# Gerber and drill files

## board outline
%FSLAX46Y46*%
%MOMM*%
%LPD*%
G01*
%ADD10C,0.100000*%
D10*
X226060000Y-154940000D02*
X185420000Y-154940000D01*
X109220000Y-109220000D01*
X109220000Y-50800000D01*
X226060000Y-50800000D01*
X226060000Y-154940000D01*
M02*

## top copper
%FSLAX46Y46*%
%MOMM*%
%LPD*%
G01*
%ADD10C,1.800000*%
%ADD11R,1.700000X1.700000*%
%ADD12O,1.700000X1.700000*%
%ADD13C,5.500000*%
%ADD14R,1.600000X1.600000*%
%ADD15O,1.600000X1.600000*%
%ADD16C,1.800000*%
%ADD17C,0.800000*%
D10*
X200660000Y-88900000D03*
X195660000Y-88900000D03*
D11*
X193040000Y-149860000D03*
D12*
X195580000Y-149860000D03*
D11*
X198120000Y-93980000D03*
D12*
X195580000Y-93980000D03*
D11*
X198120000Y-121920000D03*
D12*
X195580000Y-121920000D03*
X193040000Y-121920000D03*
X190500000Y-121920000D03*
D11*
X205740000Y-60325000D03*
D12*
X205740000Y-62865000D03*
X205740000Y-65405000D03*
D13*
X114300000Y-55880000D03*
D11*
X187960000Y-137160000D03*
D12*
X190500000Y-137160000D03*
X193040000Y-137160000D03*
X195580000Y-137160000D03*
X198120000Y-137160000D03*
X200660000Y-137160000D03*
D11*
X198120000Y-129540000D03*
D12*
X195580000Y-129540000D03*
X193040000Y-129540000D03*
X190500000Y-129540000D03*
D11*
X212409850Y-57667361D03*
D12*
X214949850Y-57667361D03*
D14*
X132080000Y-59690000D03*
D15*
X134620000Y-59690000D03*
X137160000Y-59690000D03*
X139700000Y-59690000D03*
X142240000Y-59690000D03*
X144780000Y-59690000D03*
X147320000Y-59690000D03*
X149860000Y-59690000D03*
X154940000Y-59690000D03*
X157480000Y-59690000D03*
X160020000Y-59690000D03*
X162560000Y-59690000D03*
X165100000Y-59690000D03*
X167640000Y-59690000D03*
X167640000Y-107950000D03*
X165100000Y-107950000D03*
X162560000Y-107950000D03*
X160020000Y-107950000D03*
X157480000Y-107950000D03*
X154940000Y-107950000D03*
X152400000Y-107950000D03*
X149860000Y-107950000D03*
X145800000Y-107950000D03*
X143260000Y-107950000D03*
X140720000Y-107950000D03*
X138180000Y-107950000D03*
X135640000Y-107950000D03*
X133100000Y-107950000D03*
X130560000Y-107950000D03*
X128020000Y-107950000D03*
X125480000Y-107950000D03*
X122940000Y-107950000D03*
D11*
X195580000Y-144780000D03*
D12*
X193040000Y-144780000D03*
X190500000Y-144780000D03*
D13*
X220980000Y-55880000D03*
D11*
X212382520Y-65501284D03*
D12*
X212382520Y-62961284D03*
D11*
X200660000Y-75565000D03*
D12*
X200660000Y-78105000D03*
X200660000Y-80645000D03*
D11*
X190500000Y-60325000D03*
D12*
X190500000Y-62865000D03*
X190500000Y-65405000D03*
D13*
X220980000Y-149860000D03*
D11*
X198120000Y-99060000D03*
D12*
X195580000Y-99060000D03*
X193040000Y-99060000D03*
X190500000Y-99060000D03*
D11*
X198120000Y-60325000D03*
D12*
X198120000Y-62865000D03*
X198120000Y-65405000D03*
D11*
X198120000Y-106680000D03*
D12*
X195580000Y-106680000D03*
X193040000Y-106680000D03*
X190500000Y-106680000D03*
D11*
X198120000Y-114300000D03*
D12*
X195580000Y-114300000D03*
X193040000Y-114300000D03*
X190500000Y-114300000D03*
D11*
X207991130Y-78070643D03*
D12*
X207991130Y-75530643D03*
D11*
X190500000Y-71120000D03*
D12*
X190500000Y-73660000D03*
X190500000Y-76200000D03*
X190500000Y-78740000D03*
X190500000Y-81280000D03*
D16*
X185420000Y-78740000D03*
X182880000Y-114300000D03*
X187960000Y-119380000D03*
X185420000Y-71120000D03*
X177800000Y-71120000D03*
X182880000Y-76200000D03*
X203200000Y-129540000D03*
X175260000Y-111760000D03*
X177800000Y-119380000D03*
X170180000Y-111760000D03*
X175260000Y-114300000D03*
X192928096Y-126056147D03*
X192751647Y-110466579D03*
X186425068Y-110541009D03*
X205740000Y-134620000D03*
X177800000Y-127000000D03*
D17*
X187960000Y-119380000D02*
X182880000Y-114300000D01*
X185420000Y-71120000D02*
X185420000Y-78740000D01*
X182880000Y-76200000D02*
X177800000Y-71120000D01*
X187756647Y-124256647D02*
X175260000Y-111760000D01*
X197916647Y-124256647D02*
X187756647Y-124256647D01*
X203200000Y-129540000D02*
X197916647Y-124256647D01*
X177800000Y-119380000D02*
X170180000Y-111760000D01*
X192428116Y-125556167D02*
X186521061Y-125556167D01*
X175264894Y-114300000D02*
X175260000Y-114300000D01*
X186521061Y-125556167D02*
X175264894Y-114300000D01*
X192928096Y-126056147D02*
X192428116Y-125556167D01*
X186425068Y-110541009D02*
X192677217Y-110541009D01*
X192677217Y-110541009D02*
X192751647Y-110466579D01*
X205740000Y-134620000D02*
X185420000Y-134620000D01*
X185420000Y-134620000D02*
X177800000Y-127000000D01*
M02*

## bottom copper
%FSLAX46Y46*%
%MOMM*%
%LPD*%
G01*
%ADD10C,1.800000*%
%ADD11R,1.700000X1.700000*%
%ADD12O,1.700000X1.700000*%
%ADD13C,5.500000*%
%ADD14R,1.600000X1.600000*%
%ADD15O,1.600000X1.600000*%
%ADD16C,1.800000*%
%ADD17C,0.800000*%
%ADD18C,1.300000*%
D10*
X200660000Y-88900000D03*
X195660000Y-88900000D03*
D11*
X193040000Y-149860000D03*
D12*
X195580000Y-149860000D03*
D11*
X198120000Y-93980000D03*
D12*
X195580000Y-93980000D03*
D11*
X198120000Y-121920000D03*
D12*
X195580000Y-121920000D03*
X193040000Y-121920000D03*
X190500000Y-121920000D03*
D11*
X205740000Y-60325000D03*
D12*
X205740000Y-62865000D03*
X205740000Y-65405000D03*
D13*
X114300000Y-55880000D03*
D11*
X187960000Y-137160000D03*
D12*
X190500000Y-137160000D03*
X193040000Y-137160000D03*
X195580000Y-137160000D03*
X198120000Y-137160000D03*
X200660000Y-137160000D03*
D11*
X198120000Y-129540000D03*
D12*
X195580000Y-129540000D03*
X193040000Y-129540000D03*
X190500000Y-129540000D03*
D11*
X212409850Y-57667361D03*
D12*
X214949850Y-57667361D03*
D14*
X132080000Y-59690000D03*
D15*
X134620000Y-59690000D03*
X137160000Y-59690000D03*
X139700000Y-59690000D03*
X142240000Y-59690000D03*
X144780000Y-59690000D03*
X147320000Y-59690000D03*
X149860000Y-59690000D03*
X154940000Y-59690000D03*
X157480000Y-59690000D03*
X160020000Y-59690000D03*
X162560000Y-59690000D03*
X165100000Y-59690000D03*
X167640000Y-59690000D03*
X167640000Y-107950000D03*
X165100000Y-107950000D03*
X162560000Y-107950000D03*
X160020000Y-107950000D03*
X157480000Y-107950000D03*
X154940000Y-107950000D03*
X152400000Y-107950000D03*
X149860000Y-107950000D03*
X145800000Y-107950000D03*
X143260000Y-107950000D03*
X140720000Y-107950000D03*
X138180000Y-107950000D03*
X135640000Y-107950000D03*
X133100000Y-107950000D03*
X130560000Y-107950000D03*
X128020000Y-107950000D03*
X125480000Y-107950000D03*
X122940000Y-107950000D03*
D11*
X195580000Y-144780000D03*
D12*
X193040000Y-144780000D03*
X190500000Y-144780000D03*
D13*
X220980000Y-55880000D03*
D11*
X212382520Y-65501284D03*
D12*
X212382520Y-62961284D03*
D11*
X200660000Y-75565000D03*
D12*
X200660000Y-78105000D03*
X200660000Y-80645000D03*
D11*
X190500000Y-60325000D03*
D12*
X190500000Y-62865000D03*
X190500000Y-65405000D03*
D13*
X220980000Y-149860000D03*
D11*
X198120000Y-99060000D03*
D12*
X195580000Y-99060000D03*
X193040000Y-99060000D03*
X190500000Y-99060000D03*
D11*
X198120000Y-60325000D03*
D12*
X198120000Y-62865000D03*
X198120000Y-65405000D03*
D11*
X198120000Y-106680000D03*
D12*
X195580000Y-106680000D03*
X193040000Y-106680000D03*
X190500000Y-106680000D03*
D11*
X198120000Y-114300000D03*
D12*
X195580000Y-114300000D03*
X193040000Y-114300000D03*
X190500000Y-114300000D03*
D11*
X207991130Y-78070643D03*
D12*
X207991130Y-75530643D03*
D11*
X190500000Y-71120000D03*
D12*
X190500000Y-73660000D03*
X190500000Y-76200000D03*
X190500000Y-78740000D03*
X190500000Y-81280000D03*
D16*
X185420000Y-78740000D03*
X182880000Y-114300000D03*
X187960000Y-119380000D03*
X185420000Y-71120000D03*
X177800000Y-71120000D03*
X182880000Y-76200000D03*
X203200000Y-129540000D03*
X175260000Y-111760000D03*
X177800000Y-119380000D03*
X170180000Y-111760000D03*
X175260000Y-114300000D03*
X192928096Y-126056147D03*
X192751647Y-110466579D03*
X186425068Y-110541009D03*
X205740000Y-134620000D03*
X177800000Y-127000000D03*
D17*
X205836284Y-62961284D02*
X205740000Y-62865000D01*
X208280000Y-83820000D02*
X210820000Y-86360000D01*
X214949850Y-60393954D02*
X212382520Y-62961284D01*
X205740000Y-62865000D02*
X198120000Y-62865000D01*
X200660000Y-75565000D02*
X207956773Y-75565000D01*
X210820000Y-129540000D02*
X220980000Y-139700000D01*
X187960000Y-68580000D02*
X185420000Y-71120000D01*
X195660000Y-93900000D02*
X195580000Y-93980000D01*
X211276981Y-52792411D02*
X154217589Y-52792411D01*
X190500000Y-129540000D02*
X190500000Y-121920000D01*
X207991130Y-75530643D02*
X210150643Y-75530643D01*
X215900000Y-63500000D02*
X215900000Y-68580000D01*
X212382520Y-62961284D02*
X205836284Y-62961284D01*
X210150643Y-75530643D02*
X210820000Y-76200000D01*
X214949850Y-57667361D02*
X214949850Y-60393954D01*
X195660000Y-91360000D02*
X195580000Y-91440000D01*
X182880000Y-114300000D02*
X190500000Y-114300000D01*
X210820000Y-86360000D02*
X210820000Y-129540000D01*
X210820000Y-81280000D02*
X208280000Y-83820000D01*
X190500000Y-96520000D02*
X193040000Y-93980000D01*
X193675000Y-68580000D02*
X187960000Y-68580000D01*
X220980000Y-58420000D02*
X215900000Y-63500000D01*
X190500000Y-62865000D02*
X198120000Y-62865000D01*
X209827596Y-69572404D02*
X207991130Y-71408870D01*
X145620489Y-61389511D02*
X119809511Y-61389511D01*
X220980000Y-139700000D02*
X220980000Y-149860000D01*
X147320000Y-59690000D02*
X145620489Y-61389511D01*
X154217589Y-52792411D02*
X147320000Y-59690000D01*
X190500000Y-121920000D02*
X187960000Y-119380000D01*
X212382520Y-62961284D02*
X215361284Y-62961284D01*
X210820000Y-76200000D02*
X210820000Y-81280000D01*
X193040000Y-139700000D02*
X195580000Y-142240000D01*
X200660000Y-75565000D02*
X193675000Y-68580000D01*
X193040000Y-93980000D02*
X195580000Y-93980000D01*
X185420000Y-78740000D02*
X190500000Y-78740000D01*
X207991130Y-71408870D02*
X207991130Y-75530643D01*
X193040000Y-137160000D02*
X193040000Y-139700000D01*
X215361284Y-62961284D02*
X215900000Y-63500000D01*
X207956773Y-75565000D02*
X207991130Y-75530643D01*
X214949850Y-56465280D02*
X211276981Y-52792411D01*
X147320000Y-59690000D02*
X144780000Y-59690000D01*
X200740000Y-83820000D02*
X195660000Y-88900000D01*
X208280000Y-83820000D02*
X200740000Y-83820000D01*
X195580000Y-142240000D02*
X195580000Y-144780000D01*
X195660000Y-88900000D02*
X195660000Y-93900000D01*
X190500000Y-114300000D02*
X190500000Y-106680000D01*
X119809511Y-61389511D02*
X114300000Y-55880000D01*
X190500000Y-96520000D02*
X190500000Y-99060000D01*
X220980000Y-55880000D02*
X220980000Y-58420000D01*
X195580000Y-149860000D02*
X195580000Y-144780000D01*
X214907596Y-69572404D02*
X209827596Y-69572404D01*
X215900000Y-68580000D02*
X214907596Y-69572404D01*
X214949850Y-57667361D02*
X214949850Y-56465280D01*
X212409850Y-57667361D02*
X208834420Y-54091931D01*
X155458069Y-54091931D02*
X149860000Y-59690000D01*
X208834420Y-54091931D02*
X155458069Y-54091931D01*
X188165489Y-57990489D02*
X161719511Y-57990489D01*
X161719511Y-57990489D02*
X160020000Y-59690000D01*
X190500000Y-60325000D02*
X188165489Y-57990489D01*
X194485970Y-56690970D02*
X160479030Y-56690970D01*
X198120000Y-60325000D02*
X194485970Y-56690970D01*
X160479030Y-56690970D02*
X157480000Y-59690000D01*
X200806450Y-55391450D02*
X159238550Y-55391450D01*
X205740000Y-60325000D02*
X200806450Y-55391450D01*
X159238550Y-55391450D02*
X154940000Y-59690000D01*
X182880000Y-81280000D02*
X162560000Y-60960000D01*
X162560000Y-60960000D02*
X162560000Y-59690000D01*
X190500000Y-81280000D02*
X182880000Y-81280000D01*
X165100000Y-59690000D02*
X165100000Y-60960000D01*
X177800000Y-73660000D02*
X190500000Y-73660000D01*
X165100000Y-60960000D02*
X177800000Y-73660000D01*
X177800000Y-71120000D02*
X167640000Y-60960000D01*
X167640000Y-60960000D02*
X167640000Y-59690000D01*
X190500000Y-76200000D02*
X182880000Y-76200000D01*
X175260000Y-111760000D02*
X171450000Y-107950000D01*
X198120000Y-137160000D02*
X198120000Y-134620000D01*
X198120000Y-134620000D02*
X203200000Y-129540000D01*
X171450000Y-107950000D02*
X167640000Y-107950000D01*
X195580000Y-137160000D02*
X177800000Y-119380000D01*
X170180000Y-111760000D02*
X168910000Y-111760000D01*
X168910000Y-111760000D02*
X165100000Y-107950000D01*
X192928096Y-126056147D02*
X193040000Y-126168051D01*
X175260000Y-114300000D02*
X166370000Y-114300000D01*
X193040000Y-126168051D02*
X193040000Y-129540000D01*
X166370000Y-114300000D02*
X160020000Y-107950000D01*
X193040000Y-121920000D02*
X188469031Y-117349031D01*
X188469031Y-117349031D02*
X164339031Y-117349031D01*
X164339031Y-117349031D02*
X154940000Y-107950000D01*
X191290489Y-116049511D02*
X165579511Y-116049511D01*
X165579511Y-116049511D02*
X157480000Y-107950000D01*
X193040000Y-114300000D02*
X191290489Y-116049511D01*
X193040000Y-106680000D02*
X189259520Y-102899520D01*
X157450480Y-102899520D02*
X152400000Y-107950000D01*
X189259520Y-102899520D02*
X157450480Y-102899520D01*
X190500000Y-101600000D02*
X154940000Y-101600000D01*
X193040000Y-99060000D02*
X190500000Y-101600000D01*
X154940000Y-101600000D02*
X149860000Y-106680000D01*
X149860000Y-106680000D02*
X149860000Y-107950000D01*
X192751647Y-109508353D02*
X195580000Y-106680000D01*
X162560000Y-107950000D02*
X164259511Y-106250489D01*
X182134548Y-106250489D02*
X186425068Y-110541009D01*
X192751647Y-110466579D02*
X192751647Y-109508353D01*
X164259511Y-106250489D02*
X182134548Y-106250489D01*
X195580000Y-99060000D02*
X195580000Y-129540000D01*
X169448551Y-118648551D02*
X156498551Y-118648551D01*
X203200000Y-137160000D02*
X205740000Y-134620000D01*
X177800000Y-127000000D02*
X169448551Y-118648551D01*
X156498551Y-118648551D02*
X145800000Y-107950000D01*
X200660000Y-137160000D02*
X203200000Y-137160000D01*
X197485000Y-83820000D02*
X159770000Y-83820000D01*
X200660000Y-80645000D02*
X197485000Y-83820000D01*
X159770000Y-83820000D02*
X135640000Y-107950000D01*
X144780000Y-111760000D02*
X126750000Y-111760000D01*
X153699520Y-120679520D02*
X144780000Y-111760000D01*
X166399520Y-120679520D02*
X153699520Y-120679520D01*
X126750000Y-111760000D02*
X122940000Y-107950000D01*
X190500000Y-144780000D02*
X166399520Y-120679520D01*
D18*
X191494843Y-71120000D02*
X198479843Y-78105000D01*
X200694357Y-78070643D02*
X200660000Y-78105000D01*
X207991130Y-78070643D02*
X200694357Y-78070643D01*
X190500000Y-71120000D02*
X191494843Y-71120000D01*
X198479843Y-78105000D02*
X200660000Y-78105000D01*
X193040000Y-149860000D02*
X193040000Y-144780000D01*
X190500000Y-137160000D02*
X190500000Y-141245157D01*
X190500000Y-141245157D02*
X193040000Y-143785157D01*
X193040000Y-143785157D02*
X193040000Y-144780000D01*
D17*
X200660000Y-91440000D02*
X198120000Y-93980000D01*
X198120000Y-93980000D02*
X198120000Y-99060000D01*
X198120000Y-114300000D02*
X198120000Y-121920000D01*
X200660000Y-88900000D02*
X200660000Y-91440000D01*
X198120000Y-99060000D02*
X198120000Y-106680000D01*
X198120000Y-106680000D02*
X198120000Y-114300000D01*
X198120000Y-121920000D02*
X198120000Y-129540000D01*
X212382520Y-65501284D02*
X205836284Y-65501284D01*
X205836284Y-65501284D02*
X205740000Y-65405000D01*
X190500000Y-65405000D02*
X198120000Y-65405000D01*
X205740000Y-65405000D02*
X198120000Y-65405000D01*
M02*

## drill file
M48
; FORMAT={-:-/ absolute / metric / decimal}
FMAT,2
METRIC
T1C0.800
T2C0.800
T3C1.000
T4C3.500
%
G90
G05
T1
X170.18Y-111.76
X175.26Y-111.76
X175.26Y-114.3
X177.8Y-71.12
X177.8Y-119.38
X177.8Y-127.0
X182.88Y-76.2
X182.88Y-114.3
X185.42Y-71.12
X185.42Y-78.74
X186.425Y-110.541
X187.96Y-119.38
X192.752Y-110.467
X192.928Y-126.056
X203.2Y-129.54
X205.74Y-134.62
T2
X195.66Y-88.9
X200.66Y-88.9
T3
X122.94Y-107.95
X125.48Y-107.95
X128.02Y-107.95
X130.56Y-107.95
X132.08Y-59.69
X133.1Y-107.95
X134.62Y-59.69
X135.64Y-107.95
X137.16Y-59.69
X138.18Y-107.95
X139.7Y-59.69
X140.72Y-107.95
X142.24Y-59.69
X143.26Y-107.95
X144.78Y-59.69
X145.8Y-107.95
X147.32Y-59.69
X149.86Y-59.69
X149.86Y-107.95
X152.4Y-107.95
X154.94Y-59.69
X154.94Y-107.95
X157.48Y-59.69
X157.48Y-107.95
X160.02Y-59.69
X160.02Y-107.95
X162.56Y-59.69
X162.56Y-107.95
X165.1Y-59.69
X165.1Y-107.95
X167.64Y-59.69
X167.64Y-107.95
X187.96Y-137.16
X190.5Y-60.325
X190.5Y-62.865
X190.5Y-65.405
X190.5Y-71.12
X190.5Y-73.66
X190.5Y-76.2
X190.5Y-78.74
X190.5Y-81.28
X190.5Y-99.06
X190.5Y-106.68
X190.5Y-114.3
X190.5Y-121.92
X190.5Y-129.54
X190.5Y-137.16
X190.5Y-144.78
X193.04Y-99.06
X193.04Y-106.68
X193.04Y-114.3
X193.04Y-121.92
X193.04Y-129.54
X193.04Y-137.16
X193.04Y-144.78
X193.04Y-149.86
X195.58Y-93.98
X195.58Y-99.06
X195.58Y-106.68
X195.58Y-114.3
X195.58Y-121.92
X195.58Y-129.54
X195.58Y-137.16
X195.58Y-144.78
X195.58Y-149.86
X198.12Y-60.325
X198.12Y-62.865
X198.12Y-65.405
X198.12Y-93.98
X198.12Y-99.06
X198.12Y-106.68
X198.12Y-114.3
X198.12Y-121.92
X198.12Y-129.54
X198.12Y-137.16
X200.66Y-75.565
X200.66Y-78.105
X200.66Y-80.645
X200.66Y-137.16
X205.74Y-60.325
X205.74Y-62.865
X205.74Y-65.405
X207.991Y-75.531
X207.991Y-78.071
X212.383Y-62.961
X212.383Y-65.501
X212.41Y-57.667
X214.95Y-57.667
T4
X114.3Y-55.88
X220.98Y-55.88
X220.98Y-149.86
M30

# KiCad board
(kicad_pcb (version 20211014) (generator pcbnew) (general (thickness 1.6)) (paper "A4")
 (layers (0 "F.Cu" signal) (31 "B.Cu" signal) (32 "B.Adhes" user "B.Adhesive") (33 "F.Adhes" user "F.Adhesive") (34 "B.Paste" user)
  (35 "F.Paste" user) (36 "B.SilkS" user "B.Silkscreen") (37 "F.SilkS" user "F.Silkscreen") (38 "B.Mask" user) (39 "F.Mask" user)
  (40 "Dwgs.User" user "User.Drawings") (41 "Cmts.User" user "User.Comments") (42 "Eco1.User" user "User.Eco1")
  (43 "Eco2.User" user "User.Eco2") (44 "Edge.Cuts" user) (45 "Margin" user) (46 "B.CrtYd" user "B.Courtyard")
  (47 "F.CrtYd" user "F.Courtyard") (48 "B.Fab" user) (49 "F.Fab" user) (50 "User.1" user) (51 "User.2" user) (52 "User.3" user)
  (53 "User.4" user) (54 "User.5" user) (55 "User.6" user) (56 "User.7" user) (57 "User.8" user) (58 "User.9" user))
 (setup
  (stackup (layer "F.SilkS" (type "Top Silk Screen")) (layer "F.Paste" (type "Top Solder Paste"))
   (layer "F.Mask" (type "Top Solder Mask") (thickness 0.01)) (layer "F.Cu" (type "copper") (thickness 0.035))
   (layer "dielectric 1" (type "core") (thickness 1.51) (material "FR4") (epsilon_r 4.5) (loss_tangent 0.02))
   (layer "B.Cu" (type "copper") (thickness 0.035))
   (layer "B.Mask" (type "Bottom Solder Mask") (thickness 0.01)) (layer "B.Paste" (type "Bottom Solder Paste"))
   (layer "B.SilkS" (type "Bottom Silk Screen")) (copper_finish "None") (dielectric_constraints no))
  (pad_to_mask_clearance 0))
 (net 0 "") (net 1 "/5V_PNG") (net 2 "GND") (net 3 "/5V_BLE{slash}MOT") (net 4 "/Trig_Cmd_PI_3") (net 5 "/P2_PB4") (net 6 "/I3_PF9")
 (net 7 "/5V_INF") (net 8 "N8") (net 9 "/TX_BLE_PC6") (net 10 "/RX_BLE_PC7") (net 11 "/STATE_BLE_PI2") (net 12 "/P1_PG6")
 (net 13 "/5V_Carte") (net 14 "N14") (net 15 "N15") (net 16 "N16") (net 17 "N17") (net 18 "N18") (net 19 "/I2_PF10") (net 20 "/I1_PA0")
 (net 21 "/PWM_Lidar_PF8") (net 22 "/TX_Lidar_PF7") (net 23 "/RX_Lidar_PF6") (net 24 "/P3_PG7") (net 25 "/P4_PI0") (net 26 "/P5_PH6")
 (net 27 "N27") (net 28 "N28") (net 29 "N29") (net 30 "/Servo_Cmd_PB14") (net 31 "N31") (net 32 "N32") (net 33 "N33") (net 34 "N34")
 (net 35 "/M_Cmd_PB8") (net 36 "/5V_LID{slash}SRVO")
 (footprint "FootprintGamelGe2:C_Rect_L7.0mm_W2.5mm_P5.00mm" (layer "F.Cu") (at 200.66 88.9 180)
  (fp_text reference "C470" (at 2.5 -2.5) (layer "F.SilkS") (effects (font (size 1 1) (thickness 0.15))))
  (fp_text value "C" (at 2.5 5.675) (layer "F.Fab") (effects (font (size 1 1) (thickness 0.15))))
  (pad "1" thru_hole circle locked (at 0 0 180) (size 1.8 1.8) (drill 0.8) (layers *.Cu *.Mask) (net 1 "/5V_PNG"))
  (pad "2" thru_hole circle locked (at 5 0 180) (size 1.8 1.8) (drill 0.8) (layers *.Cu *.Mask) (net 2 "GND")))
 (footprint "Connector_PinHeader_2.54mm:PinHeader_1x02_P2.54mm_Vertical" (layer "F.Cu") (at 193.04 149.86 90)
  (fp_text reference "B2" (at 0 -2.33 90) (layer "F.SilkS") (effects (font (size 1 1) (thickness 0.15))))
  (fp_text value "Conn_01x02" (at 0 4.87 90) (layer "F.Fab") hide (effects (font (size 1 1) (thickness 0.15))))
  (pad "1" thru_hole rect (at 0 0 90) (size 1.7 1.7) (drill 1) (layers *.Cu *.Mask) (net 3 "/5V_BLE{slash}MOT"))
  (pad "2" thru_hole oval (at 0 2.54 90) (size 1.7 1.7) (drill 1) (layers *.Cu *.Mask) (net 2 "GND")))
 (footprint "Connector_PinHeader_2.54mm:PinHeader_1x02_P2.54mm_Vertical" (layer "F.Cu") (at 198.12 93.98 -90)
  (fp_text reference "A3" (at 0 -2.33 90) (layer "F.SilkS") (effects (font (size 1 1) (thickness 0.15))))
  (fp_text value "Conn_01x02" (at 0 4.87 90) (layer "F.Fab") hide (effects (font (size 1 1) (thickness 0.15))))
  (pad "1" thru_hole rect (at 0 0 270) (size 1.7 1.7) (drill 1) (layers *.Cu *.Mask) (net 1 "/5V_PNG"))
  (pad "2" thru_hole oval (at 0 2.54 270) (size 1.7 1.7) (drill 1) (layers *.Cu *.Mask) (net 2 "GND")))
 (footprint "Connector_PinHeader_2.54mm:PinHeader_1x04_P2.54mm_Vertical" (layer "F.Cu") (at 198.12 121.92 -90)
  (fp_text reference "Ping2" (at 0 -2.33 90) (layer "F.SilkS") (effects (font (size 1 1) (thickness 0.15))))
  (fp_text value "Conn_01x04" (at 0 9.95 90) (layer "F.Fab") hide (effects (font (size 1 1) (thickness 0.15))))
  (pad "1" thru_hole rect (at 0 0 270) (size 1.7 1.7) (drill 1) (layers *.Cu *.Mask) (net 1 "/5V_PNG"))
  (pad "2" thru_hole oval (at 0 2.54 270) (size 1.7 1.7) (drill 1) (layers *.Cu *.Mask) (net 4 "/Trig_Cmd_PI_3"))
  (pad "3" thru_hole oval (at 0 5.08 270) (size 1.7 1.7) (drill 1) (layers *.Cu *.Mask) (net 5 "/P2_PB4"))
  (pad "4" thru_hole oval (at 0 7.62 270) (size 1.7 1.7) (drill 1) (layers *.Cu *.Mask) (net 2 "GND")))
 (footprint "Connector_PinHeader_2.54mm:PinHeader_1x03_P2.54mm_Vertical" (layer "F.Cu") (at 205.74 60.325)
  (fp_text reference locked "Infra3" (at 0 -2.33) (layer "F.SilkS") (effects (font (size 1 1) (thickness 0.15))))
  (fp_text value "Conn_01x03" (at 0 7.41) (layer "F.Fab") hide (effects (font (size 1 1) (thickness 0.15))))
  (pad "1" thru_hole rect (at 0 0) (size 1.7 1.7) (drill 1) (layers *.Cu *.Mask) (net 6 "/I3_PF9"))
  (pad "2" thru_hole oval (at 0 2.54) (size 1.7 1.7) (drill 1) (layers *.Cu *.Mask) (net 2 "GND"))
  (pad "3" thru_hole oval (at 0 5.08) (size 1.7 1.7) (drill 1) (layers *.Cu *.Mask) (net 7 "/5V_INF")))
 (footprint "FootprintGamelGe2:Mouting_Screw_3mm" (layer "F.Cu") (at 114.3 55.88)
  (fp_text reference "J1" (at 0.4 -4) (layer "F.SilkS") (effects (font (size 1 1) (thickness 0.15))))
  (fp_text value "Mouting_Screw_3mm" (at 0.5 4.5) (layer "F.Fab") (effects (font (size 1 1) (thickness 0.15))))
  (pad "1" thru_hole circle locked (at 0 0) (size 5.5 5.5) (drill 3.5) (layers *.Cu *.Mask) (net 2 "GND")))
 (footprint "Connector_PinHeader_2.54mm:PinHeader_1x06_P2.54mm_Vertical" (layer "F.Cu") (at 187.96 137.16 90)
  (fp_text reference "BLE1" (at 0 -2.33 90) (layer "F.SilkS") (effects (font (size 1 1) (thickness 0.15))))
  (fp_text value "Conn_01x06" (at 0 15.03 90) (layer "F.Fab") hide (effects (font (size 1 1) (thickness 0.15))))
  (pad "1" thru_hole rect (at 0 0 90) (size 1.7 1.7) (drill 1) (layers *.Cu *.Mask) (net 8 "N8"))
  (pad "2" thru_hole oval (at 0 2.54 90) (size 1.7 1.7) (drill 1) (layers *.Cu *.Mask) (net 3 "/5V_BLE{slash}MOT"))
  (pad "3" thru_hole oval (at 0 5.08 90) (size 1.7 1.7) (drill 1) (layers *.Cu *.Mask) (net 2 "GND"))
  (pad "4" thru_hole oval (at 0 7.62 90) (size 1.7 1.7) (drill 1) (layers *.Cu *.Mask) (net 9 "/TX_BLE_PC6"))
  (pad "5" thru_hole oval (at 0 10.16 90) (size 1.7 1.7) (drill 1) (layers *.Cu *.Mask) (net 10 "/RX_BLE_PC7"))
  (pad "6" thru_hole oval (at 0 12.7 90) (size 1.7 1.7) (drill 1) (layers *.Cu *.Mask) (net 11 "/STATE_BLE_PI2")))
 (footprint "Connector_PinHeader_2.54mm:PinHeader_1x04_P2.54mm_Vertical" (layer "F.Cu") (at 198.12 129.54 -90)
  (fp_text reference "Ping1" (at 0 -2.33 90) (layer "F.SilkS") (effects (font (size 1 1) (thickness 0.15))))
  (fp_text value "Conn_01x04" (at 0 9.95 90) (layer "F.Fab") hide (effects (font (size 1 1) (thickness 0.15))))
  (pad "1" thru_hole rect (at 0 0 270) (size 1.7 1.7) (drill 1) (layers *.Cu *.Mask) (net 1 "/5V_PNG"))
  (pad "2" thru_hole oval (at 0 2.54 270) (size 1.7 1.7) (drill 1) (layers *.Cu *.Mask) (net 4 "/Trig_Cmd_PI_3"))
  (pad "3" thru_hole oval (at 0 5.08 270) (size 1.7 1.7) (drill 1) (layers *.Cu *.Mask) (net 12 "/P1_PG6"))
  (pad "4" thru_hole oval (at 0 7.62 270) (size 1.7 1.7) (drill 1) (layers *.Cu *.Mask) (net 2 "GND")))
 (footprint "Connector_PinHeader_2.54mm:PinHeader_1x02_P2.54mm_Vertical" (layer "F.Cu") (at 212.40985 57.667361 90)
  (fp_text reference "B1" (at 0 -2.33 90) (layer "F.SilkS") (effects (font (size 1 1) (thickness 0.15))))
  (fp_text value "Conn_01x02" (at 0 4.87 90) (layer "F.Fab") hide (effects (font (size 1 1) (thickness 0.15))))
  (pad "1" thru_hole rect (at 0 0 90) (size 1.7 1.7) (drill 1) (layers *.Cu *.Mask) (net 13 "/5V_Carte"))
  (pad "2" thru_hole oval (at 0 2.54 90) (size 1.7 1.7) (drill 1) (layers *.Cu *.Mask) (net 2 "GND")))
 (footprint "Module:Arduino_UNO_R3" (layer "F.Cu") (at 132.08 59.69)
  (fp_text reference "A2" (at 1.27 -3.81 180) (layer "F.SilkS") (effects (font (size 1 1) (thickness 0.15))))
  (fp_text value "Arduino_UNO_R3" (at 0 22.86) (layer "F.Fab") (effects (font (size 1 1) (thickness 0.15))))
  (pad "1" thru_hole rect (at 0 0 90) (size 1.6 1.6) (drill 1) (layers *.Cu *.Mask) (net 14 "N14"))
  (pad "2" thru_hole oval (at 2.54 0 90) (size 1.6 1.6) (drill 1) (layers *.Cu *.Mask) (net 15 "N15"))
  (pad "3" thru_hole oval (at 5.08 0 90) (size 1.6 1.6) (drill 1) (layers *.Cu *.Mask) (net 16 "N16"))
  (pad "4" thru_hole oval (at 7.62 0 90) (size 1.6 1.6) (drill 1) (layers *.Cu *.Mask) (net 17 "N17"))
  (pad "5" thru_hole oval (at 10.16 0 90) (size 1.6 1.6) (drill 1) (layers *.Cu *.Mask) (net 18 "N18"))
  (pad "6" thru_hole oval (at 12.7 0 90) (size 1.6 1.6) (drill 1) (layers *.Cu *.Mask) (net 2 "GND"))
  (pad "7" thru_hole oval (at 15.24 0 90) (size 1.6 1.6) (drill 1) (layers *.Cu *.Mask) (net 2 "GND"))
  (pad "8" thru_hole oval (at 17.78 0 90) (size 1.6 1.6) (drill 1) (layers *.Cu *.Mask) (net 13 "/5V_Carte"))
  (pad "9" thru_hole oval (at 22.86 0 90) (size 1.6 1.6) (drill 1) (layers *.Cu *.Mask) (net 6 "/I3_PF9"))
  (pad "10" thru_hole oval (at 25.4 0 90) (size 1.6 1.6) (drill 1) (layers *.Cu *.Mask) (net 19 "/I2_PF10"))
  (pad "11" thru_hole oval (at 27.94 0 90) (size 1.6 1.6) (drill 1) (layers *.Cu *.Mask) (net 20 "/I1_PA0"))
  (pad "12" thru_hole oval (at 30.48 0 90) (size 1.6 1.6) (drill 1) (layers *.Cu *.Mask) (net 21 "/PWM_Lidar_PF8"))
  (pad "13" thru_hole oval (at 33.02 0 90) (size 1.6 1.6) (drill 1) (layers *.Cu *.Mask) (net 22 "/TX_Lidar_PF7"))
  (pad "14" thru_hole oval (at 35.56 0 90) (size 1.6 1.6) (drill 1) (layers *.Cu *.Mask) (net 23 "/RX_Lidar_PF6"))
  (pad "15" thru_hole oval (at 35.56 48.26 90) (size 1.6 1.6) (drill 1) (layers *.Cu *.Mask) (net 10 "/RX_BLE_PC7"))
  (pad "16" thru_hole oval (at 33.02 48.26 90) (size 1.6 1.6) (drill 1) (layers *.Cu *.Mask) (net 9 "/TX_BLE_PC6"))
  (pad "17" thru_hole oval (at 30.48 48.26 90) (size 1.6 1.6) (drill 1) (layers *.Cu *.Mask) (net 4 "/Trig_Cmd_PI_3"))
  (pad "18" thru_hole oval (at 27.94 48.26 90) (size 1.6 1.6) (drill 1) (layers *.Cu *.Mask) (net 12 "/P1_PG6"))
  (pad "19" thru_hole oval (at 25.4 48.26 90) (size 1.6 1.6) (drill 1) (layers *.Cu *.Mask) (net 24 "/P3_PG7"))
  (pad "20" thru_hole oval (at 22.86 48.26 90) (size 1.6 1.6) (drill 1) (layers *.Cu *.Mask) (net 5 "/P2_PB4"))
  (pad "21" thru_hole oval (at 20.32 48.26 90) (size 1.6 1.6) (drill 1) (layers *.Cu *.Mask) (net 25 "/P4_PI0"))
  (pad "22" thru_hole oval (at 17.78 48.26 90) (size 1.6 1.6) (drill 1) (layers *.Cu *.Mask) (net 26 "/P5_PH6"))
  (pad "23" thru_hole oval (at 13.72 48.26 90) (size 1.6 1.6) (drill 1) (layers *.Cu *.Mask) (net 11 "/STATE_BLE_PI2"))
  (pad "24" thru_hole oval (at 11.18 48.26 90) (size 1.6 1.6) (drill 1) (layers *.Cu *.Mask) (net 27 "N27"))
  (pad "25" thru_hole oval (at 8.64 48.26 90) (size 1.6 1.6) (drill 1) (layers *.Cu *.Mask) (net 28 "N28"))
  (pad "26" thru_hole oval (at 6.1 48.26 90) (size 1.6 1.6) (drill 1) (layers *.Cu *.Mask) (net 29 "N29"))
  (pad "27" thru_hole oval (at 3.56 48.26 90) (size 1.6 1.6) (drill 1) (layers *.Cu *.Mask) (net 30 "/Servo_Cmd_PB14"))
  (pad "28" thru_hole oval (at 1.02 48.26 90) (size 1.6 1.6) (drill 1) (layers *.Cu *.Mask) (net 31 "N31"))
  (pad "29" thru_hole oval (at -1.52 48.26 90) (size 1.6 1.6) (drill 1) (layers *.Cu *.Mask) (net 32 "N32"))
  (pad "30" thru_hole oval (at -4.06 48.26 90) (size 1.6 1.6) (drill 1) (layers *.Cu *.Mask) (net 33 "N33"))
  (pad "31" thru_hole oval (at -6.6 48.26 90) (size 1.6 1.6) (drill 1) (layers *.Cu *.Mask) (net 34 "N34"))
  (pad "32" thru_hole oval (at -9.14 48.26 90) (size 1.6 1.6) (drill 1) (layers *.Cu *.Mask) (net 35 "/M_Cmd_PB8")))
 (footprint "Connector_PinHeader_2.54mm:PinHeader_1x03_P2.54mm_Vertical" (layer "F.Cu") (at 195.58 144.78 -90)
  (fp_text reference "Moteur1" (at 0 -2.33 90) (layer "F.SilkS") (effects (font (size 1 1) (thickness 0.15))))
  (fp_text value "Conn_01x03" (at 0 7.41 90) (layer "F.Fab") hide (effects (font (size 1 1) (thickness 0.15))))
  (pad "1" thru_hole rect (at 0 0 270) (size 1.7 1.7) (drill 1) (layers *.Cu *.Mask) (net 2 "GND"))
  (pad "2" thru_hole oval (at 0 2.54 270) (size 1.7 1.7) (drill 1) (layers *.Cu *.Mask) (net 3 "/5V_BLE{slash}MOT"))
  (pad "3" thru_hole oval (at 0 5.08 270) (size 1.7 1.7) (drill 1) (layers *.Cu *.Mask) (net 35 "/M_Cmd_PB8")))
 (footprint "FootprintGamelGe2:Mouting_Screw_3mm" (layer "F.Cu") (at 220.98 55.88)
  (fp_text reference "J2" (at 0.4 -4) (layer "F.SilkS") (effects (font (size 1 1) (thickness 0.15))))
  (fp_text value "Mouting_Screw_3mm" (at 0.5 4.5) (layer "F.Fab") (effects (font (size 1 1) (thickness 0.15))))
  (pad "1" thru_hole circle locked (at 0 0) (size 5.5 5.5) (drill 3.5) (layers *.Cu *.Mask) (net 2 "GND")))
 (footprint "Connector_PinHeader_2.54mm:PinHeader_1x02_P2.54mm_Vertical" (layer "F.Cu") (at 212.38252 65.501284 180)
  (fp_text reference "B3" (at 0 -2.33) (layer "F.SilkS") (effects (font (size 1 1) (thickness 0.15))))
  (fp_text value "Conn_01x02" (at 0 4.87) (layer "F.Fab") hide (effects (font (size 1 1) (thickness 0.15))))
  (pad "1" thru_hole rect (at 0 0 180) (size 1.7 1.7) (drill 1) (layers *.Cu *.Mask) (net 7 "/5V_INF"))
  (pad "2" thru_hole oval (at 0 2.54 180) (size 1.7 1.7) (drill 1) (layers *.Cu *.Mask) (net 2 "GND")))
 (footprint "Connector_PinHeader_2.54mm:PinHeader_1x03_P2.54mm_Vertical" (layer "F.Cu") (at 200.66 75.565)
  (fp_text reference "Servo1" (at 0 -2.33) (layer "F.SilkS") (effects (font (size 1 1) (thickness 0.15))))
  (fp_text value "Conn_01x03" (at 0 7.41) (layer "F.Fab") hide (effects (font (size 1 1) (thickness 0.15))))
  (pad "1" thru_hole rect (at 0 0) (size 1.7 1.7) (drill 1) (layers *.Cu *.Mask) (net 2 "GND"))
  (pad "2" thru_hole oval (at 0 2.54) (size 1.7 1.7) (drill 1) (layers *.Cu *.Mask) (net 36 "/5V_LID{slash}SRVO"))
  (pad "3" thru_hole oval (at 0 5.08) (size 1.7 1.7) (drill 1) (layers *.Cu *.Mask) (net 30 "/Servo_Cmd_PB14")))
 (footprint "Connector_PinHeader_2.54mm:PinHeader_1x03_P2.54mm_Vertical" (layer "F.Cu") (at 190.5 60.325)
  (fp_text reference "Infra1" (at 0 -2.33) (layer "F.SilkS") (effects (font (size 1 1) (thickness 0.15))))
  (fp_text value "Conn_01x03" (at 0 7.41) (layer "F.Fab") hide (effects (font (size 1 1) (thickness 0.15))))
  (pad "1" thru_hole rect (at 0 0) (size 1.7 1.7) (drill 1) (layers *.Cu *.Mask) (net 20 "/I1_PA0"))
  (pad "2" thru_hole oval (at 0 2.54) (size 1.7 1.7) (drill 1) (layers *.Cu *.Mask) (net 2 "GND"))
  (pad "3" thru_hole oval (at 0 5.08) (size 1.7 1.7) (drill 1) (layers *.Cu *.Mask) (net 7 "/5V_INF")))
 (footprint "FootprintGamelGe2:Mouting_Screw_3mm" (layer "F.Cu") (at 220.98 149.86)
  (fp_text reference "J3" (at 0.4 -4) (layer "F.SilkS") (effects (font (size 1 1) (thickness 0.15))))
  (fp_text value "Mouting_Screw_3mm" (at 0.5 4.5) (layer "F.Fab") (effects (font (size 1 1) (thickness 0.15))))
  (pad "1" thru_hole circle locked (at 0 0) (size 5.5 5.5) (drill 3.5) (layers *.Cu *.Mask) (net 2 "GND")))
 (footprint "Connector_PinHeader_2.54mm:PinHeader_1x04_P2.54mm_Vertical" (layer "F.Cu") (at 198.12 99.06 -90)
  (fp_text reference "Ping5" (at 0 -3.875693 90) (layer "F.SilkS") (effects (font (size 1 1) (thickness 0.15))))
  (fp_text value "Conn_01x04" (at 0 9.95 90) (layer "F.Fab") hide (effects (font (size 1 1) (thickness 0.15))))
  (pad "1" thru_hole rect (at 0 0 270) (size 1.7 1.7) (drill 1) (layers *.Cu *.Mask) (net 1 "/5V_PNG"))
  (pad "2" thru_hole oval (at 0 2.54 270) (size 1.7 1.7) (drill 1) (layers *.Cu *.Mask) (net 4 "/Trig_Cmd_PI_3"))
  (pad "3" thru_hole oval (at 0 5.08 270) (size 1.7 1.7) (drill 1) (layers *.Cu *.Mask) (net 26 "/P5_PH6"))
  (pad "4" thru_hole oval (at 0 7.62 270) (size 1.7 1.7) (drill 1) (layers *.Cu *.Mask) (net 2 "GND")))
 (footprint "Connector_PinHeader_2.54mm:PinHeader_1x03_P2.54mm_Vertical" (layer "F.Cu") (at 198.12 60.325)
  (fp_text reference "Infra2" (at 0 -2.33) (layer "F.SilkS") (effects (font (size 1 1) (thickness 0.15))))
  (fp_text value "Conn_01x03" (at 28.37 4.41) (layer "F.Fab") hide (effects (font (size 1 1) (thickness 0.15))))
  (pad "1" thru_hole rect (at 0 0) (size 1.7 1.7) (drill 1) (layers *.Cu *.Mask) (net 19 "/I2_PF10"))
  (pad "2" thru_hole oval (at 0 2.54) (size 1.7 1.7) (drill 1) (layers *.Cu *.Mask) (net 2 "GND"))
  (pad "3" thru_hole oval (at 0 5.08) (size 1.7 1.7) (drill 1) (layers *.Cu *.Mask) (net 7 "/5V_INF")))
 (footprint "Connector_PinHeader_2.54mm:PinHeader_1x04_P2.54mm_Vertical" (layer "F.Cu") (at 198.12 106.68 -90)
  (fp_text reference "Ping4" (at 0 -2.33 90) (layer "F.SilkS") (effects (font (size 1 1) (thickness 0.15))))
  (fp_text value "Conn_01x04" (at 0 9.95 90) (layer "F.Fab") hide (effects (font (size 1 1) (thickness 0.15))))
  (pad "1" thru_hole rect (at 0 0 270) (size 1.7 1.7) (drill 1) (layers *.Cu *.Mask) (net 1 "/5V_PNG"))
  (pad "2" thru_hole oval (at 0 2.54 270) (size 1.7 1.7) (drill 1) (layers *.Cu *.Mask) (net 4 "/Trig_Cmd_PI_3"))
  (pad "3" thru_hole oval (at 0 5.08 270) (size 1.7 1.7) (drill 1) (layers *.Cu *.Mask) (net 25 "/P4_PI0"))
  (pad "4" thru_hole oval (at 0 7.62 270) (size 1.7 1.7) (drill 1) (layers *.Cu *.Mask) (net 2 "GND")))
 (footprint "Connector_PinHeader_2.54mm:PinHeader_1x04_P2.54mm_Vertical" (layer "F.Cu") (at 198.12 114.3 -90)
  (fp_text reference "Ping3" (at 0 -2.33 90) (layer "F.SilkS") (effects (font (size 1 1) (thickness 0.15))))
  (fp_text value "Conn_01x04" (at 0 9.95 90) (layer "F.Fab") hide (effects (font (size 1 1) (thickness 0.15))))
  (pad "1" thru_hole rect (at 0 0 270) (size 1.7 1.7) (drill 1) (layers *.Cu *.Mask) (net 1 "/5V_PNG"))
  (pad "2" thru_hole oval (at 0 2.54 270) (size 1.7 1.7) (drill 1) (layers *.Cu *.Mask) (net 4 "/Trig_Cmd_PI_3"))
  (pad "3" thru_hole oval (at 0 5.08 270) (size 1.7 1.7) (drill 1) (layers *.Cu *.Mask) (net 24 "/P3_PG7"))
  (pad "4" thru_hole oval (at 0 7.62 270) (size 1.7 1.7) (drill 1) (layers *.Cu *.Mask) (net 2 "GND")))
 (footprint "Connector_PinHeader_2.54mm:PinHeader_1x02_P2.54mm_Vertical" (layer "F.Cu") (at 207.99113 78.070643 180)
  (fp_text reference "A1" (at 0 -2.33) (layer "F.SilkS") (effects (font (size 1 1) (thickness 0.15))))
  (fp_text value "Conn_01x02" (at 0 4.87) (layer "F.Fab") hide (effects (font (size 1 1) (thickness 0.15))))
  (pad "1" thru_hole rect (at 0 0 180) (size 1.7 1.7) (drill 1) (layers *.Cu *.Mask) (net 36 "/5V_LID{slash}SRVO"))
  (pad "2" thru_hole oval (at 0 2.54 180) (size 1.7 1.7) (drill 1) (layers *.Cu *.Mask) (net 2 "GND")))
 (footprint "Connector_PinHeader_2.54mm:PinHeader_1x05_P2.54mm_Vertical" (layer "F.Cu") (at 190.5 71.12)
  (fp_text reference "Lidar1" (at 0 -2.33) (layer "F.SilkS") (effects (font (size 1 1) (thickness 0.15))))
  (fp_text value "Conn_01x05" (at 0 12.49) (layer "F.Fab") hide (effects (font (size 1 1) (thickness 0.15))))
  (pad "1" thru_hole rect (at 0 0) (size 1.7 1.7) (drill 1) (layers *.Cu *.Mask) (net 36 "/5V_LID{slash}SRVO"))
  (pad "2" thru_hole oval (at 0 2.54) (size 1.7 1.7) (drill 1) (layers *.Cu *.Mask) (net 22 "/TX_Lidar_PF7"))
  (pad "3" thru_hole oval (at 0 5.08) (size 1.7 1.7) (drill 1) (layers *.Cu *.Mask) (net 23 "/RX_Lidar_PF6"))
  (pad "4" thru_hole oval (at 0 7.62) (size 1.7 1.7) (drill 1) (layers *.Cu *.Mask) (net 2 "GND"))
  (pad "5" thru_hole oval (at 0 10.16) (size 1.7 1.7) (drill 1) (layers *.Cu *.Mask) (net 21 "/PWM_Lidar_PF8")))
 (gr_poly
  (pts (xy 226.06 154.94) (xy 185.42 154.94) (xy 109.22 109.22) (xy 109.22 50.8) (xy 226.06 50.8)) (layer "Edge.Cuts") (width 0.1)
  (fill none))
 (segment (start 187.96 119.38) (end 182.88 114.3) (width 0.8) (layer "F.Cu") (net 2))
 (segment (start 185.42 71.12) (end 185.42 78.74) (width 0.8) (layer "F.Cu") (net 2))
 (via (at 185.42 78.74) (size 1.8) (drill 0.8) (layers "F.Cu" "B.Cu") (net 2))
 (via (at 182.88 114.3) (size 1.8) (drill 0.8) (layers "F.Cu" "B.Cu") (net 2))
 (via (at 187.96 119.38) (size 1.8) (drill 0.8) (layers "F.Cu" "B.Cu") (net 2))
 (via (at 185.42 71.12) (size 1.8) (drill 0.8) (layers "F.Cu" "B.Cu") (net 2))
 (segment (start 205.836284 62.961284) (end 205.74 62.865) (width 0.8) (layer "B.Cu") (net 2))
 (segment (start 208.28 83.82) (end 210.82 86.36) (width 0.8) (layer "B.Cu") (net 2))
 (segment (start 214.94985 60.393954) (end 212.38252 62.961284) (width 0.8) (layer "B.Cu") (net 2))
 (segment (start 205.74 62.865) (end 198.12 62.865) (width 0.8) (layer "B.Cu") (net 2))
 (segment (start 200.66 75.565) (end 207.956773 75.565) (width 0.8) (layer "B.Cu") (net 2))
 (segment (start 210.82 129.54) (end 220.98 139.7) (width 0.8) (layer "B.Cu") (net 2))
 (segment (start 187.96 68.58) (end 185.42 71.12) (width 0.8) (layer "B.Cu") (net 2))
 (segment (start 195.66 93.9) (end 195.58 93.98) (width 0.8) (layer "B.Cu") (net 2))
 (segment (start 211.276981 52.792411) (end 154.217589 52.792411) (width 0.8) (layer "B.Cu") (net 2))
 (segment (start 190.5 129.54) (end 190.5 121.92) (width 0.8) (layer "B.Cu") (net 2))
 (segment (start 207.99113 75.530643) (end 210.150643 75.530643) (width 0.8) (layer "B.Cu") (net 2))
 (segment (start 215.9 63.5) (end 215.9 68.58) (width 0.8) (layer "B.Cu") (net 2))
 (segment (start 212.38252 62.961284) (end 205.836284 62.961284) (width 0.8) (layer "B.Cu") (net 2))
 (segment (start 210.150643 75.530643) (end 210.82 76.2) (width 0.8) (layer "B.Cu") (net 2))
 (segment (start 214.94985 57.667361) (end 214.94985 60.393954) (width 0.8) (layer "B.Cu") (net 2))
 (segment (start 195.66 91.36) (end 195.58 91.44) (width 0.8) (layer "B.Cu") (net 2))
 (segment (start 182.88 114.3) (end 190.5 114.3) (width 0.8) (layer "B.Cu") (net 2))
 (segment (start 210.82 86.36) (end 210.82 129.54) (width 0.8) (layer "B.Cu") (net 2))
 (segment (start 210.82 81.28) (end 208.28 83.82) (width 0.8) (layer "B.Cu") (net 2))
 (segment (start 190.5 96.52) (end 193.04 93.98) (width 0.8) (layer "B.Cu") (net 2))
 (segment (start 193.675 68.58) (end 187.96 68.58) (width 0.8) (layer "B.Cu") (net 2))
 (segment (start 220.98 58.42) (end 215.9 63.5) (width 0.8) (layer "B.Cu") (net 2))
 (segment (start 190.5 62.865) (end 198.12 62.865) (width 0.8) (layer "B.Cu") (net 2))
 (segment (start 209.827596 69.572404) (end 207.99113 71.40887) (width 0.8) (layer "B.Cu") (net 2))
 (segment (start 145.620489 61.389511) (end 119.809511 61.389511) (width 0.8) (layer "B.Cu") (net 2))
 (segment (start 220.98 139.7) (end 220.98 149.86) (width 0.8) (layer "B.Cu") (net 2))
 (segment (start 147.32 59.69) (end 145.620489 61.389511) (width 0.8) (layer "B.Cu") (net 2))
 (segment (start 154.217589 52.792411) (end 147.32 59.69) (width 0.8) (layer "B.Cu") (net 2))
 (segment (start 190.5 121.92) (end 187.96 119.38) (width 0.8) (layer "B.Cu") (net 2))
 (segment (start 212.38252 62.961284) (end 215.361284 62.961284) (width 0.8) (layer "B.Cu") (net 2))
 (segment (start 210.82 76.2) (end 210.82 81.28) (width 0.8) (layer "B.Cu") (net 2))
 (segment (start 193.04 139.7) (end 195.58 142.24) (width 0.8) (layer "B.Cu") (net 2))
 (segment (start 200.66 75.565) (end 193.675 68.58) (width 0.8) (layer "B.Cu") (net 2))
 (segment (start 193.04 93.98) (end 195.58 93.98) (width 0.8) (layer "B.Cu") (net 2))
 (segment (start 185.42 78.74) (end 190.5 78.74) (width 0.8) (layer "B.Cu") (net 2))
 (segment (start 207.99113 71.40887) (end 207.99113 75.530643) (width 0.8) (layer "B.Cu") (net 2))
 (segment (start 193.04 137.16) (end 193.04 139.7) (width 0.8) (layer "B.Cu") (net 2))
 (segment (start 215.361284 62.961284) (end 215.9 63.5) (width 0.8) (layer "B.Cu") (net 2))
 (segment (start 207.956773 75.565) (end 207.99113 75.530643) (width 0.8) (layer "B.Cu") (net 2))
 (segment (start 214.94985 56.46528) (end 211.276981 52.792411) (width 0.8) (layer "B.Cu") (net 2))
 (segment (start 147.32 59.69) (end 144.78 59.69) (width 0.8) (layer "B.Cu") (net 2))
 (segment (start 200.74 83.82) (end 195.66 88.9) (width 0.8) (layer "B.Cu") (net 2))
 (segment (start 208.28 83.82) (end 200.74 83.82) (width 0.8) (layer "B.Cu") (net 2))
 (segment (start 195.58 142.24) (end 195.58 144.78) (width 0.8) (layer "B.Cu") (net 2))
 (segment (start 195.66 88.9) (end 195.66 93.9) (width 0.8) (layer "B.Cu") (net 2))
 (segment (start 190.5 114.3) (end 190.5 106.68) (width 0.8) (layer "B.Cu") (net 2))
 (segment (start 119.809511 61.389511) (end 114.3 55.88) (width 0.8) (layer "B.Cu") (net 2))
 (segment (start 190.5 96.52) (end 190.5 99.06) (width 0.8) (layer "B.Cu") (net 2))
 (segment (start 220.98 55.88) (end 220.98 58.42) (width 0.8) (layer "B.Cu") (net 2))
 (segment (start 195.58 149.86) (end 195.58 144.78) (width 0.8) (layer "B.Cu") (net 2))
 (segment (start 214.907596 69.572404) (end 209.827596 69.572404) (width 0.8) (layer "B.Cu") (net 2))
 (segment (start 215.9 68.58) (end 214.907596 69.572404) (width 0.8) (layer "B.Cu") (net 2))
 (segment (start 214.94985 57.667361) (end 214.94985 56.46528) (width 0.8) (layer "B.Cu") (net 2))
 (segment (start 212.40985 57.667361) (end 208.83442 54.091931) (width 0.8) (layer "B.Cu") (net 13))
 (segment (start 155.458069 54.091931) (end 149.86 59.69) (width 0.8) (layer "B.Cu") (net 13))
 (segment (start 208.83442 54.091931) (end 155.458069 54.091931) (width 0.8) (layer "B.Cu") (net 13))
 (segment (start 188.165489 57.990489) (end 161.719511 57.990489) (width 0.8) (layer "B.Cu") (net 20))
 (segment (start 161.719511 57.990489) (end 160.02 59.69) (width 0.8) (layer "B.Cu") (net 20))
 (segment (start 190.5 60.325) (end 188.165489 57.990489) (width 0.8) (layer "B.Cu") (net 20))
 (segment (start 194.48597 56.69097) (end 160.47903 56.69097) (width 0.8) (layer "B.Cu") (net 19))
 (segment (start 198.12 60.325) (end 194.48597 56.69097) (width 0.8) (layer "B.Cu") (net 19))
 (segment (start 160.47903 56.69097) (end 157.48 59.69) (width 0.8) (layer "B.Cu") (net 19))
 (segment (start 200.80645 55.39145) (end 159.23855 55.39145) (width 0.8) (layer "B.Cu") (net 6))
 (segment (start 205.74 60.325) (end 200.80645 55.39145) (width 0.8) (layer "B.Cu") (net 6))
 (segment (start 159.23855 55.39145) (end 154.94 59.69) (width 0.8) (layer "B.Cu") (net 6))
 (segment (start 182.88 81.28) (end 162.56 60.96) (width 0.8) (layer "B.Cu") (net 21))
 (segment (start 162.56 60.96) (end 162.56 59.69) (width 0.8) (layer "B.Cu") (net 21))
 (segment (start 190.5 81.28) (end 182.88 81.28) (width 0.8) (layer "B.Cu") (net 21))
 (segment (start 165.1 59.69) (end 165.1 60.96) (width 0.8) (layer "B.Cu") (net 22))
 (segment (start 177.8 73.66) (end 190.5 73.66) (width 0.8) (layer "B.Cu") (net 22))
 (segment (start 165.1 60.96) (end 177.8 73.66) (width 0.8) (layer "B.Cu") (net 22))
 (segment (start 182.88 76.2) (end 177.8 71.12) (width 0.8) (layer "F.Cu") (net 23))
 (via (at 177.8 71.12) (size 1.8) (drill 0.8) (layers "F.Cu" "B.Cu") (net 23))
 (via (at 182.88 76.2) (size 1.8) (drill 0.8) (layers "F.Cu" "B.Cu") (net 23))
 (segment (start 177.8 71.12) (end 167.64 60.96) (width 0.8) (layer "B.Cu") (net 23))
 (segment (start 167.64 60.96) (end 167.64 59.69) (width 0.8) (layer "B.Cu") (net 23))
 (segment (start 190.5 76.2) (end 182.88 76.2) (width 0.8) (layer "B.Cu") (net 23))
 (segment (start 187.756647 124.256647) (end 175.26 111.76) (width 0.8) (layer "F.Cu") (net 10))
 (segment (start 197.916647 124.256647) (end 187.756647 124.256647) (width 0.8) (layer "F.Cu") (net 10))
 (segment (start 203.2 129.54) (end 197.916647 124.256647) (width 0.8) (layer "F.Cu") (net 10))
 (via (at 203.2 129.54) (size 1.8) (drill 0.8) (layers "F.Cu" "B.Cu") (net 10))
 (via (at 175.26 111.76) (size 1.8) (drill 0.8) (layers "F.Cu" "B.Cu") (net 10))
 (segment (start 175.26 111.76) (end 171.45 107.95) (width 0.8) (layer "B.Cu") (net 10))
 (segment (start 198.12 137.16) (end 198.12 134.62) (width 0.8) (layer "B.Cu") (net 10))
 (segment (start 198.12 134.62) (end 203.2 129.54) (width 0.8) (layer "B.Cu") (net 10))
 (segment (start 171.45 107.95) (end 167.64 107.95) (width 0.8) (layer "B.Cu") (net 10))
 (segment (start 177.8 119.38) (end 170.18 111.76) (width 0.8) (layer "F.Cu") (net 9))
 (via (at 177.8 119.38) (size 1.8) (drill 0.8) (layers "F.Cu" "B.Cu") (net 9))
 (via (at 170.18 111.76) (size 1.8) (drill 0.8) (layers "F.Cu" "B.Cu") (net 9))
 (segment (start 195.58 137.16) (end 177.8 119.38) (width 0.8) (layer "B.Cu") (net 9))
 (segment (start 170.18 111.76) (end 168.91 111.76) (width 0.8) (layer "B.Cu") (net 9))
 (segment (start 168.91 111.76) (end 165.1 107.95) (width 0.8) (layer "B.Cu") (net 9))
 (segment (start 192.428116 125.556167) (end 186.521061 125.556167) (width 0.8) (layer "F.Cu") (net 12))
 (segment (start 175.264894 114.3) (end 175.26 114.3) (width 0.8) (layer "F.Cu") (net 12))
 (segment (start 186.521061 125.556167) (end 175.264894 114.3) (width 0.8) (layer "F.Cu") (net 12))
 (segment (start 192.928096 126.056147) (end 192.428116 125.556167) (width 0.8) (layer "F.Cu") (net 12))
 (via (at 175.26 114.3) (size 1.8) (drill 0.8) (layers "F.Cu" "B.Cu") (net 12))
 (via (at 192.928096 126.056147) (size 1.8) (drill 0.8) (layers "F.Cu" "B.Cu") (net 12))
 (segment (start 192.928096 126.056147) (end 193.04 126.168051) (width 0.8) (layer "B.Cu") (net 12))
 (segment (start 175.26 114.3) (end 166.37 114.3) (width 0.8) (layer "B.Cu") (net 12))
 (segment (start 193.04 126.168051) (end 193.04 129.54) (width 0.8) (layer "B.Cu") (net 12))
 (segment (start 166.37 114.3) (end 160.02 107.95) (width 0.8) (layer "B.Cu") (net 12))
 (segment (start 193.04 121.92) (end 188.469031 117.349031) (width 0.8) (layer "B.Cu") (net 5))
 (segment (start 188.469031 117.349031) (end 164.339031 117.349031) (width 0.8) (layer "B.Cu") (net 5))
 (segment (start 164.339031 117.349031) (end 154.94 107.95) (width 0.8) (layer "B.Cu") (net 5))
 (segment (start 191.290489 116.049511) (end 165.579511 116.049511) (width 0.8) (layer "B.Cu") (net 24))
 (segment (start 165.579511 116.049511) (end 157.48 107.95) (width 0.8) (layer "B.Cu") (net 24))
 (segment (start 193.04 114.3) (end 191.290489 116.049511) (width 0.8) (layer "B.Cu") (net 24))
 (segment (start 193.04 106.68) (end 189.25952 102.89952) (width 0.8) (layer "B.Cu") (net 25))
 (segment (start 157.45048 102.89952) (end 152.4 107.95) (width 0.8) (layer "B.Cu") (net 25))
 (segment (start 189.25952 102.89952) (end 157.45048 102.89952) (width 0.8) (layer "B.Cu") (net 25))
 (segment (start 190.5 101.6) (end 154.94 101.6) (width 0.8) (layer "B.Cu") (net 26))
 (segment (start 193.04 99.06) (end 190.5 101.6) (width 0.8) (layer "B.Cu") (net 26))
 (segment (start 154.94 101.6) (end 149.86 106.68) (width 0.8) (layer "B.Cu") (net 26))
 (segment (start 149.86 106.68) (end 149.86 107.95) (width 0.8) (layer "B.Cu") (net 26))
 (segment (start 186.425068 110.541009) (end 192.677217 110.541009) (width 0.8) (layer "F.Cu") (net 4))
 (segment (start 192.677217 110.541009) (end 192.751647 110.466579) (width 0.8) (layer "F.Cu") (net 4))
 (via (at 192.751647 110.466579) (size 1.8) (drill 0.8) (layers "F.Cu" "B.Cu") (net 4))
 (via (at 186.425068 110.541009) (size 1.8) (drill 0.8) (layers "F.Cu" "B.Cu") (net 4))
 (segment (start 192.751647 109.508353) (end 195.58 106.68) (width 0.8) (layer "B.Cu") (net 4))
 (segment (start 162.56 107.95) (end 164.259511 106.250489) (width 0.8) (layer "B.Cu") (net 4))
 (segment (start 182.134548 106.250489) (end 186.425068 110.541009) (width 0.8) (layer "B.Cu") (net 4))
 (segment (start 192.751647 110.466579) (end 192.751647 109.508353) (width 0.8) (layer "B.Cu") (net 4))
 (segment (start 164.259511 106.250489) (end 182.134548 106.250489) (width 0.8) (layer "B.Cu") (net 4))
 (segment (start 195.58 99.06) (end 195.58 129.54) (width 0.8) (layer "B.Cu") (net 4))
 (segment (start 205.74 134.62) (end 185.42 134.62) (width 0.8) (layer "F.Cu") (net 11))
 (segment (start 185.42 134.62) (end 177.8 127) (width 0.8) (layer "F.Cu") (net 11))
 (via (at 205.74 134.62) (size 1.8) (drill 0.8) (layers "F.Cu" "B.Cu") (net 11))
 (via (at 177.8 127) (size 1.8) (drill 0.8) (layers "F.Cu" "B.Cu") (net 11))
 (segment (start 169.448551 118.648551) (end 156.498551 118.648551) (width 0.8) (layer "B.Cu") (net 11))
 (segment (start 203.2 137.16) (end 205.74 134.62) (width 0.8) (layer "B.Cu") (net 11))
 (segment (start 177.8 127) (end 169.448551 118.648551) (width 0.8) (layer "B.Cu") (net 11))
 (segment (start 156.498551 118.648551) (end 145.8 107.95) (width 0.8) (layer "B.Cu") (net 11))
 (segment (start 200.66 137.16) (end 203.2 137.16) (width 0.8) (layer "B.Cu") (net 11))
 (segment (start 197.485 83.82) (end 159.77 83.82) (width 0.8) (layer "B.Cu") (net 30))
 (segment (start 200.66 80.645) (end 197.485 83.82) (width 0.8) (layer "B.Cu") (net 30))
 (segment (start 159.77 83.82) (end 135.64 107.95) (width 0.8) (layer "B.Cu") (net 30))
 (segment (start 144.78 111.76) (end 126.75 111.76) (width 0.8) (layer "B.Cu") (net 35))
 (segment (start 153.69952 120.67952) (end 144.78 111.76) (width 0.8) (layer "B.Cu") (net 35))
 (segment (start 166.39952 120.67952) (end 153.69952 120.67952) (width 0.8) (layer "B.Cu") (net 35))
 (segment (start 126.75 111.76) (end 122.94 107.95) (width 0.8) (layer "B.Cu") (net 35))
 (segment (start 190.5 144.78) (end 166.39952 120.67952) (width 0.8) (layer "B.Cu") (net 35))
 (segment (start 191.494843 71.12) (end 198.479843 78.105) (width 1.3) (layer "B.Cu") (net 36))
 (segment (start 200.694357 78.070643) (end 200.66 78.105) (width 1.3) (layer "B.Cu") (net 36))
 (segment (start 207.99113 78.070643) (end 200.694357 78.070643) (width 1.3) (layer "B.Cu") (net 36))
 (segment (start 190.5 71.12) (end 191.494843 71.12) (width 1.3) (layer "B.Cu") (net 36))
 (segment (start 198.479843 78.105) (end 200.66 78.105) (width 1.3) (layer "B.Cu") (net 36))
 (segment (start 193.04 149.86) (end 193.04 144.78) (width 1.3) (layer "B.Cu") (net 3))
 (segment (start 190.5 137.16) (end 190.5 141.245157) (width 1.3) (layer "B.Cu") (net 3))
 (segment (start 190.5 141.245157) (end 193.04 143.785157) (width 1.3) (layer "B.Cu") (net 3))
 (segment (start 193.04 143.785157) (end 193.04 144.78) (width 1.3) (layer "B.Cu") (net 3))
 (segment (start 200.66 91.44) (end 198.12 93.98) (width 0.8) (layer "B.Cu") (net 1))
 (segment (start 198.12 93.98) (end 198.12 99.06) (width 0.8) (layer "B.Cu") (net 1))
 (segment (start 198.12 114.3) (end 198.12 121.92) (width 0.8) (layer "B.Cu") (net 1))
 (segment (start 200.66 88.9) (end 200.66 91.44) (width 0.8) (layer "B.Cu") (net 1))
 (segment (start 198.12 99.06) (end 198.12 106.68) (width 0.8) (layer "B.Cu") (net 1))
 (segment (start 198.12 106.68) (end 198.12 114.3) (width 0.8) (layer "B.Cu") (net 1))
 (segment (start 198.12 121.92) (end 198.12 129.54) (width 0.8) (layer "B.Cu") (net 1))
 (segment (start 212.38252 65.501284) (end 205.836284 65.501284) (width 0.8) (layer "B.Cu") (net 7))
 (segment (start 205.836284 65.501284) (end 205.74 65.405) (width 0.8) (layer "B.Cu") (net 7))
 (segment (start 190.5 65.405) (end 198.12 65.405) (width 0.8) (layer "B.Cu") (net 7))
 (segment (start 205.74 65.405) (end 198.12 65.405) (width 0.8) (layer "B.Cu") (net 7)))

